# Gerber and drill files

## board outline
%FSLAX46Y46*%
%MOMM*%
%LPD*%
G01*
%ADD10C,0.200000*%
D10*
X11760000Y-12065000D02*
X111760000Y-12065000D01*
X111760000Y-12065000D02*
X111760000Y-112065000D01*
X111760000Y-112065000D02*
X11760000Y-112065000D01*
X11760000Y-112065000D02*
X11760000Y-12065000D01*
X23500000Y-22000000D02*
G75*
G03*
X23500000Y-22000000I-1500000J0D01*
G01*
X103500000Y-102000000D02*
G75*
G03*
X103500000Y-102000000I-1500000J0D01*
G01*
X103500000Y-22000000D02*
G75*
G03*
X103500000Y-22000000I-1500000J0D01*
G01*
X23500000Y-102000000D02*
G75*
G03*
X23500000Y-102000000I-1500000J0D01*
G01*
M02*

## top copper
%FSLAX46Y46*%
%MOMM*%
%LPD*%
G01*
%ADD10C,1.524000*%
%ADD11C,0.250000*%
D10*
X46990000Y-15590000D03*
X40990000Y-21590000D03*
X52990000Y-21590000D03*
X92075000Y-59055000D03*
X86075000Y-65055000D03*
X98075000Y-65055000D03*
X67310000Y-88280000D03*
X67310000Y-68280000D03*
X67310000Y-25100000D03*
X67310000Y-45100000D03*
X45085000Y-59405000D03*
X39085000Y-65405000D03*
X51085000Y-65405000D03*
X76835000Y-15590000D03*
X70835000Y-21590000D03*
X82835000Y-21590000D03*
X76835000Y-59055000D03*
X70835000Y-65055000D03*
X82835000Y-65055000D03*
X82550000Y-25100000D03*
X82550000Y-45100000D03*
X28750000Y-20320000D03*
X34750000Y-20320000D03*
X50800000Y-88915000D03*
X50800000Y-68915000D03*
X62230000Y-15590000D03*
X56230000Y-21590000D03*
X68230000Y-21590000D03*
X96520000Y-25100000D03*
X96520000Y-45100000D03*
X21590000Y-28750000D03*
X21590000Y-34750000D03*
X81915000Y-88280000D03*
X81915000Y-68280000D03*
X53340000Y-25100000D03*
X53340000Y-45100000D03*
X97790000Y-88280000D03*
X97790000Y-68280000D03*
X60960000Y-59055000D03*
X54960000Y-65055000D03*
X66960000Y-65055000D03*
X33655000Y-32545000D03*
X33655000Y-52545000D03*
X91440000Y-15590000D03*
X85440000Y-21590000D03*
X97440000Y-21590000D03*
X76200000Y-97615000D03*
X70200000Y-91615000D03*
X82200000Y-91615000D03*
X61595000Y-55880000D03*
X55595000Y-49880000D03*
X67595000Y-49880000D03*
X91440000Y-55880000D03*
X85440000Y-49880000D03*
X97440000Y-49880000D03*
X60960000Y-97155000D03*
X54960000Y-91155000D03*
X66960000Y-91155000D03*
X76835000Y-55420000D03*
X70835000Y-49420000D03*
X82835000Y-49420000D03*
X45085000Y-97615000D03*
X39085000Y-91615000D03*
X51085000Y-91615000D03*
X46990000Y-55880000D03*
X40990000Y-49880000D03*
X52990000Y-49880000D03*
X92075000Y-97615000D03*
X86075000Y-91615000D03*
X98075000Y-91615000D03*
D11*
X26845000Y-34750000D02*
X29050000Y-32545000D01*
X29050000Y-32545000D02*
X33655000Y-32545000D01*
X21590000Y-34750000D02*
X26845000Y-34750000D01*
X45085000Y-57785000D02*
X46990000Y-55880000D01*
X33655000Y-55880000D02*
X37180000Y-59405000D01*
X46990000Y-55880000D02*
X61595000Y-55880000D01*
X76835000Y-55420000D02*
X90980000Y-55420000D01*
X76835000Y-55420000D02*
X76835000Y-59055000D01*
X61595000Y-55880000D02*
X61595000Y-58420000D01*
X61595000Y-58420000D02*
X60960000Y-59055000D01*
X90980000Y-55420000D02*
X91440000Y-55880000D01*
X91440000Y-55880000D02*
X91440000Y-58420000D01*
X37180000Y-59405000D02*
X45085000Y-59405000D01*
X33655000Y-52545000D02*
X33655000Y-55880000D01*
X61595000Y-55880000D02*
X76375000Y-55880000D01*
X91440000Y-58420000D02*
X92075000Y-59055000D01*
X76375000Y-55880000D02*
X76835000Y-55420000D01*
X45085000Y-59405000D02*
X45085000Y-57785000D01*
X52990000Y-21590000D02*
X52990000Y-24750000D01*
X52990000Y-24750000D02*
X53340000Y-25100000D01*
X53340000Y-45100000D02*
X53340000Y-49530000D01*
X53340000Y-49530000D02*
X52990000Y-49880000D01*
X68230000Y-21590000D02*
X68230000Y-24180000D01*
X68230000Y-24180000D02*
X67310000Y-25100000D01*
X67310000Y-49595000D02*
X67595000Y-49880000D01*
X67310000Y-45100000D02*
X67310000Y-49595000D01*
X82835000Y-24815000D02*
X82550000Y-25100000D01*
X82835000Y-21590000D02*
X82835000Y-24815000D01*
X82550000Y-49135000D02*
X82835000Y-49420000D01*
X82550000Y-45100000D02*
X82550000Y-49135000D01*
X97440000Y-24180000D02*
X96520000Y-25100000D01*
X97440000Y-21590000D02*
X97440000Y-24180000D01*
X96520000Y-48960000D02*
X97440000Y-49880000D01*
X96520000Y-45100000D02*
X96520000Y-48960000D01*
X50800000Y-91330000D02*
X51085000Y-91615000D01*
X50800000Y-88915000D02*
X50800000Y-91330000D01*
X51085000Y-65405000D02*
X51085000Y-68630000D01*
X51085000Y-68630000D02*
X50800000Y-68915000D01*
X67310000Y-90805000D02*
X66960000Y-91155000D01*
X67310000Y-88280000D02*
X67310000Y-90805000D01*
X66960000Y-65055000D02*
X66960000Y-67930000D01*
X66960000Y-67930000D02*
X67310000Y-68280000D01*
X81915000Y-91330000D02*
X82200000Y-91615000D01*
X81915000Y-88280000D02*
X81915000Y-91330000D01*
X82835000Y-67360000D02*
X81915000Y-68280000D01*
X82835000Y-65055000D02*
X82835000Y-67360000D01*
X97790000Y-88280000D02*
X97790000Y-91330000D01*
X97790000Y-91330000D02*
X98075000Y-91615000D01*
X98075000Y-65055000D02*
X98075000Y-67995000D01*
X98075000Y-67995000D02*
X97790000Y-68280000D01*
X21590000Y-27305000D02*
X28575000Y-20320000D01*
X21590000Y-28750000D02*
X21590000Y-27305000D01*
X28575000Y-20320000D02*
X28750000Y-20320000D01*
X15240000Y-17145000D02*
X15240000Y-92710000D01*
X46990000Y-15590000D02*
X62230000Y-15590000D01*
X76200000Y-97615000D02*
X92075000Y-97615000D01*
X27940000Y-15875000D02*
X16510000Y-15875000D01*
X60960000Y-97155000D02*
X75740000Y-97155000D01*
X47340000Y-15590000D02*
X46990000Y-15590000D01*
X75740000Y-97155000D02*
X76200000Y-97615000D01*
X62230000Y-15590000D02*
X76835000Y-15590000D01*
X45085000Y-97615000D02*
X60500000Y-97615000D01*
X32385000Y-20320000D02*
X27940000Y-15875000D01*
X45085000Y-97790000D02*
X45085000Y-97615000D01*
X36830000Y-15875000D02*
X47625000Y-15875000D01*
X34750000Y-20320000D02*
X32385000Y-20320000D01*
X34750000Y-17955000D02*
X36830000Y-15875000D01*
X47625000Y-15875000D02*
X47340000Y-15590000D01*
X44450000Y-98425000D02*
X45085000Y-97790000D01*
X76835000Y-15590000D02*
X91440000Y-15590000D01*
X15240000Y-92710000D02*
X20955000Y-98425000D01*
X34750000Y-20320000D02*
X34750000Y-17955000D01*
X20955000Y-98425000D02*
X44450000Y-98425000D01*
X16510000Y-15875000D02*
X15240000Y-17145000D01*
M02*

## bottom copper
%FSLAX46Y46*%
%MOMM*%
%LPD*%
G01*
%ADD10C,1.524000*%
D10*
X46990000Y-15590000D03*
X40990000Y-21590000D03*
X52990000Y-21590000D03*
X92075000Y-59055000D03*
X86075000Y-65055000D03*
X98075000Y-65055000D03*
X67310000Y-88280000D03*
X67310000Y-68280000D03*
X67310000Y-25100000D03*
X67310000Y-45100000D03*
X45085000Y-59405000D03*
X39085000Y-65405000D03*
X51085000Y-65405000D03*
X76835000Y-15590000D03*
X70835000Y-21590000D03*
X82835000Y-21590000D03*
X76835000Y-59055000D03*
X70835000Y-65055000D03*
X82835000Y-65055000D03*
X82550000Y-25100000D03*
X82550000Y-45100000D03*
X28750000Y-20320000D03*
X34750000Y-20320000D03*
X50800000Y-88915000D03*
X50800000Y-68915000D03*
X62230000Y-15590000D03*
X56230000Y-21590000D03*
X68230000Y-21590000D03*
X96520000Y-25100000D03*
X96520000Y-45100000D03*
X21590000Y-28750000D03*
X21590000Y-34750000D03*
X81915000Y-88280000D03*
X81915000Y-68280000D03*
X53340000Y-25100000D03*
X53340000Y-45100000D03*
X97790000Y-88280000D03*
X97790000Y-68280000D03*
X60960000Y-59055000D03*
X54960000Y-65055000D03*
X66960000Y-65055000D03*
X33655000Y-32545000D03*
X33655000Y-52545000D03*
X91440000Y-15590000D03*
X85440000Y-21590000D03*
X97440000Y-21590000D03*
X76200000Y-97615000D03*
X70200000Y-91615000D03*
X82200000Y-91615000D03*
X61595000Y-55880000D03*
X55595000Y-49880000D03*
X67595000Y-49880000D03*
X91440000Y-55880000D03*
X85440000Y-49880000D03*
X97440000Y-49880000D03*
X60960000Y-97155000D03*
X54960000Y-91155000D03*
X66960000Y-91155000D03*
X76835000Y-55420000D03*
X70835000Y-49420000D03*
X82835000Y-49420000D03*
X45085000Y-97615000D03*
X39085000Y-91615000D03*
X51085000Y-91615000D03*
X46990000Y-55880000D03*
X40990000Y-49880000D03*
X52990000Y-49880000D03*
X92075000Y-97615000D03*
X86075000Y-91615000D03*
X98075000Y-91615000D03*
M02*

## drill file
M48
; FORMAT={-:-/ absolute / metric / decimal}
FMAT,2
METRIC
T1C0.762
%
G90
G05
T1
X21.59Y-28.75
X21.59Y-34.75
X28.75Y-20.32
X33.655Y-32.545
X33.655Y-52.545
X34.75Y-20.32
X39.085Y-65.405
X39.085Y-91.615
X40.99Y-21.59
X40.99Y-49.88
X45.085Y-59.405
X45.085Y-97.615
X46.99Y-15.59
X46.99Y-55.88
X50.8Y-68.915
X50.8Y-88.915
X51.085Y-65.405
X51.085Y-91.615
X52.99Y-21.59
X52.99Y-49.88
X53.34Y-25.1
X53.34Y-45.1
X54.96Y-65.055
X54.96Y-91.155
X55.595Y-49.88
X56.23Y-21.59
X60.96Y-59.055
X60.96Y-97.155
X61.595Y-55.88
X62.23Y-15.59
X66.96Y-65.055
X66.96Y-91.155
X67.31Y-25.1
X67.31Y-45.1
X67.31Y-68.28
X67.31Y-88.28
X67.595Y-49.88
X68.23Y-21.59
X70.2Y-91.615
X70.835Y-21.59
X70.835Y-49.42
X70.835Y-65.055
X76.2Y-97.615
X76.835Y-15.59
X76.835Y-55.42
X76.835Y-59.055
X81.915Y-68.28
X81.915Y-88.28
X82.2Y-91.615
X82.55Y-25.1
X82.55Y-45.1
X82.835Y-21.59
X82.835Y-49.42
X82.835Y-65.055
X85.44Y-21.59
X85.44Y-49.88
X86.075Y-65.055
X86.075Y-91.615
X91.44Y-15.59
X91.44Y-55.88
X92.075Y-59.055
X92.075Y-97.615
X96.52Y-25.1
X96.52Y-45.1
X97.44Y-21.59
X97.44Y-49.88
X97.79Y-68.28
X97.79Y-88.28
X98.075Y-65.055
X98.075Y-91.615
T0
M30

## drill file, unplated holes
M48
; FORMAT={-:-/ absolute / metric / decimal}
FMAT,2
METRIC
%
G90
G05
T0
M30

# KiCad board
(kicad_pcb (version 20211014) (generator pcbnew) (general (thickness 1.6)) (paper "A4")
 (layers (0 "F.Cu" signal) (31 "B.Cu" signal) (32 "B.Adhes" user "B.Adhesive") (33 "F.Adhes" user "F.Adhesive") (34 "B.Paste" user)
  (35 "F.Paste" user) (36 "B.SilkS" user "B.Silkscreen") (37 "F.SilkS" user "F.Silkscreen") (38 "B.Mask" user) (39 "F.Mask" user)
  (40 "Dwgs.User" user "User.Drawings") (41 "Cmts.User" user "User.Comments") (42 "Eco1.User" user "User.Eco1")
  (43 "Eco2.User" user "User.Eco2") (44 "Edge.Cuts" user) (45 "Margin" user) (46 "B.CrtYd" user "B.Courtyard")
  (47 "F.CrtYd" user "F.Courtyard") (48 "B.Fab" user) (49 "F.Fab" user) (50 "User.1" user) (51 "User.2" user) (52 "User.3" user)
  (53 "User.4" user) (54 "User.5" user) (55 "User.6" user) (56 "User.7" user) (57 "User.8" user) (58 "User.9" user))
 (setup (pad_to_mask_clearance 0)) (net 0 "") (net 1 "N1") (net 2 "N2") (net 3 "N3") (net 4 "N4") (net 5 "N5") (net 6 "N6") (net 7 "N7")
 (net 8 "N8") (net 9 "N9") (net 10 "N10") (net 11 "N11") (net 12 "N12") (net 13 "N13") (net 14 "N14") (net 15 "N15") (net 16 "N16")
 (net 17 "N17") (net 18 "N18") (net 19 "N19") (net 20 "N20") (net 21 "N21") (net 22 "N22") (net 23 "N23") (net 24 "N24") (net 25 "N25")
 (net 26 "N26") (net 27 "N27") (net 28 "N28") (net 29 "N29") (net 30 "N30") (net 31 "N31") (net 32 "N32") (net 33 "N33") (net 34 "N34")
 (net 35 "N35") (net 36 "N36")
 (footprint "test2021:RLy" (layer "F.Cu") (at 46.99 21.59)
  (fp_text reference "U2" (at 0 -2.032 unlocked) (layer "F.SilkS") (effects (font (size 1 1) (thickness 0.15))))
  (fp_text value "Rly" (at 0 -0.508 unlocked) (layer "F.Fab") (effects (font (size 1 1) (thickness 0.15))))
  (pad "1" thru_hole circle (at 0 -6) (size 1.524 1.524) (drill 0.762) (layers *.Cu *.Mask) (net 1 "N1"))
  (pad "2" thru_hole circle (at -6 0) (size 1.524 1.524) (drill 0.762) (layers *.Cu *.Mask) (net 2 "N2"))
  (pad "3" thru_hole circle (at 6 0) (size 1.524 1.524) (drill 0.762) (layers *.Cu *.Mask) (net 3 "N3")))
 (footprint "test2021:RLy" (layer "F.Cu") (at 92.075 65.055)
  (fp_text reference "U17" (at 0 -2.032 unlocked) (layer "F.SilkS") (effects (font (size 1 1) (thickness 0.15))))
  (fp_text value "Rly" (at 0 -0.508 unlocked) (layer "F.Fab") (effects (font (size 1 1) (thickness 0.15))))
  (pad "1" thru_hole circle (at 0 -6) (size 1.524 1.524) (drill 0.762) (layers *.Cu *.Mask) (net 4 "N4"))
  (pad "2" thru_hole circle (at -6 0) (size 1.524 1.524) (drill 0.762) (layers *.Cu *.Mask) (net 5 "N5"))
  (pad "3" thru_hole circle (at 6 0) (size 1.524 1.524) (drill 0.762) (layers *.Cu *.Mask) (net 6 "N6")))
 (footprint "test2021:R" (layer "F.Cu") (at 67.31 78.28 90)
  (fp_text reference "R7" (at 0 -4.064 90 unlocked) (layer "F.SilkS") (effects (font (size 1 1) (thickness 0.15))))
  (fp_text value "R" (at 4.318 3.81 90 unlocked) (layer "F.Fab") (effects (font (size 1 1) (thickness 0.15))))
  (pad "1" thru_hole circle (at -10 0 90) (size 1.524 1.524) (drill 0.762) (layers *.Cu *.Mask) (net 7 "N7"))
  (pad "2" thru_hole circle (at 10 0 90) (size 1.524 1.524) (drill 0.762) (layers *.Cu *.Mask) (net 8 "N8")))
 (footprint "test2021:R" (layer "F.Cu") (at 67.31 35.1 -90)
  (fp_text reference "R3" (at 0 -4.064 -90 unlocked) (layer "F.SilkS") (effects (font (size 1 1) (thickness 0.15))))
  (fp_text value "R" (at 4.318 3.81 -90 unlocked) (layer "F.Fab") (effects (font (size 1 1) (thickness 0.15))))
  (pad "1" thru_hole circle (at -10 0 270) (size 1.524 1.524) (drill 0.762) (layers *.Cu *.Mask) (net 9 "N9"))
  (pad "2" thru_hole circle (at 10 0 270) (size 1.524 1.524) (drill 0.762) (layers *.Cu *.Mask) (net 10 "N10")))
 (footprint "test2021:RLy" (layer "F.Cu") (at 45.085 65.405)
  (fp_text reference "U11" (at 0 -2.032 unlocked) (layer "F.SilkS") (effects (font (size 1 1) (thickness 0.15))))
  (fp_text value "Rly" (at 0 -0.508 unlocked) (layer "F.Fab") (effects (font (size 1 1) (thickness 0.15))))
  (pad "1" thru_hole circle (at 0 -6) (size 1.524 1.524) (drill 0.762) (layers *.Cu *.Mask) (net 4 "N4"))
  (pad "2" thru_hole circle (at -6 0) (size 1.524 1.524) (drill 0.762) (layers *.Cu *.Mask) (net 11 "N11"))
  (pad "3" thru_hole circle (at 6 0) (size 1.524 1.524) (drill 0.762) (layers *.Cu *.Mask) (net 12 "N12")))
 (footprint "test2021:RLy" (layer "F.Cu") (at 76.835 21.59)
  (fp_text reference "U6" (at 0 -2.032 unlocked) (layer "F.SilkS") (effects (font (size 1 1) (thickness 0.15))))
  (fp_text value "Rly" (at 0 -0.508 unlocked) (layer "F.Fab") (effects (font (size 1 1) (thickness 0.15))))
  (pad "1" thru_hole circle (at 0 -6) (size 1.524 1.524) (drill 0.762) (layers *.Cu *.Mask) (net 1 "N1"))
  (pad "2" thru_hole circle (at -6 0) (size 1.524 1.524) (drill 0.762) (layers *.Cu *.Mask) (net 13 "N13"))
  (pad "3" thru_hole circle (at 6 0) (size 1.524 1.524) (drill 0.762) (layers *.Cu *.Mask) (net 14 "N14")))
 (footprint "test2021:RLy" (layer "F.Cu") (at 76.835 65.055)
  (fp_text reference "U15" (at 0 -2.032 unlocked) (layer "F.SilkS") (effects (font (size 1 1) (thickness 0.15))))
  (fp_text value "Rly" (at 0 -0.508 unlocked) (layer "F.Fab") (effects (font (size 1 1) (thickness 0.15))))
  (pad "1" thru_hole circle (at 0 -6) (size 1.524 1.524) (drill 0.762) (layers *.Cu *.Mask) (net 4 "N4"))
  (pad "2" thru_hole circle (at -6 0) (size 1.524 1.524) (drill 0.762) (layers *.Cu *.Mask) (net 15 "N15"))
  (pad "3" thru_hole circle (at 6 0) (size 1.524 1.524) (drill 0.762) (layers *.Cu *.Mask) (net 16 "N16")))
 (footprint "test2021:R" (layer "F.Cu") (at 82.55 35.1 -90)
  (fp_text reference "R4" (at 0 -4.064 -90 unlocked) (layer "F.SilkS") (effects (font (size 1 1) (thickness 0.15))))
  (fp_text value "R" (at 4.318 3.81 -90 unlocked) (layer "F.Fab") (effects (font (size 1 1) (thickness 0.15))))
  (pad "1" thru_hole circle (at -10 0 270) (size 1.524 1.524) (drill 0.762) (layers *.Cu *.Mask) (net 14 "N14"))
  (pad "2" thru_hole circle (at 10 0 270) (size 1.524 1.524) (drill 0.762) (layers *.Cu *.Mask) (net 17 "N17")))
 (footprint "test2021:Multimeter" (layer "F.Cu") (at 31.75 20.32 90)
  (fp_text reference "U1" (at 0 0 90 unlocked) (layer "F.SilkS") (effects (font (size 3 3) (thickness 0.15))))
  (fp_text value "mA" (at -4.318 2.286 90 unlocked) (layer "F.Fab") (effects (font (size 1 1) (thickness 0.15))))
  (pad "1" thru_hole circle (at 0 -3 90) (size 1.524 1.524) (drill 0.762) (layers *.Cu *.Mask) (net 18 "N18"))
  (pad "2" thru_hole circle (at 0 3 90) (size 1.524 1.524) (drill 0.762) (layers *.Cu *.Mask) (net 1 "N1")))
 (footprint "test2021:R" (layer "F.Cu") (at 50.8 78.915 90)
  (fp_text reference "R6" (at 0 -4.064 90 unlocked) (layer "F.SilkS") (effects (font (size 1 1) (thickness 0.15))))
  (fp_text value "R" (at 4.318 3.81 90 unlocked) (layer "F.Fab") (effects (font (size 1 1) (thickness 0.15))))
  (pad "1" thru_hole circle (at -10 0 90) (size 1.524 1.524) (drill 0.762) (layers *.Cu *.Mask) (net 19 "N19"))
  (pad "2" thru_hole circle (at 10 0 90) (size 1.524 1.524) (drill 0.762) (layers *.Cu *.Mask) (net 12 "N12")))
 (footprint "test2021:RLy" (layer "F.Cu") (at 62.23 21.59)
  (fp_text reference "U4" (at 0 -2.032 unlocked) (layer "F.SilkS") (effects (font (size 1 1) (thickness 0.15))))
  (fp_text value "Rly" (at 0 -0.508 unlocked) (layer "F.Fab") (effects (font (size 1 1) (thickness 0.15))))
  (pad "1" thru_hole circle (at 0 -6) (size 1.524 1.524) (drill 0.762) (layers *.Cu *.Mask) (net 1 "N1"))
  (pad "2" thru_hole circle (at -6 0) (size 1.524 1.524) (drill 0.762) (layers *.Cu *.Mask) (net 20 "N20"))
  (pad "3" thru_hole circle (at 6 0) (size 1.524 1.524) (drill 0.762) (layers *.Cu *.Mask) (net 9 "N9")))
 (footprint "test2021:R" (layer "F.Cu") (at 96.52 35.1 -90)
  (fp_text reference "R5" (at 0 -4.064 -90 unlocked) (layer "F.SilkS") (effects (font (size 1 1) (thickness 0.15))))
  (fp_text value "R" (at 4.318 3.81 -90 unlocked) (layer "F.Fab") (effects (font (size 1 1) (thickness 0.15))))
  (pad "1" thru_hole circle (at -10 0 270) (size 1.524 1.524) (drill 0.762) (layers *.Cu *.Mask) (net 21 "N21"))
  (pad "2" thru_hole circle (at 10 0 270) (size 1.524 1.524) (drill 0.762) (layers *.Cu *.Mask) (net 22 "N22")))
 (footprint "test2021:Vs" (layer "F.Cu") (at 21.59 31.75)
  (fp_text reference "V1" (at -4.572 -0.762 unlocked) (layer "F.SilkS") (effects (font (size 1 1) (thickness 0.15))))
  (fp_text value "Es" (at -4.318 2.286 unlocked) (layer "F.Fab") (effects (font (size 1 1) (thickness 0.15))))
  (pad "1" thru_hole circle (at 0 -3) (size 1.524 1.524) (drill 0.762) (layers *.Cu *.Mask) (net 18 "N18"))
  (pad "2" thru_hole circle (at 0 3) (size 1.524 1.524) (drill 0.762) (layers *.Cu *.Mask) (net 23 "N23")))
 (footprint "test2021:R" (layer "F.Cu") (at 81.915 78.28 90)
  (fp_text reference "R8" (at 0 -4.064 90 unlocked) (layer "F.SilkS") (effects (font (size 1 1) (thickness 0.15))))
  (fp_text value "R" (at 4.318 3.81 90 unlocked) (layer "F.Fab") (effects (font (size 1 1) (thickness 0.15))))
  (pad "1" thru_hole circle (at -10 0 90) (size 1.524 1.524) (drill 0.762) (layers *.Cu *.Mask) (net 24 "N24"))
  (pad "2" thru_hole circle (at 10 0 90) (size 1.524 1.524) (drill 0.762) (layers *.Cu *.Mask) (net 16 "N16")))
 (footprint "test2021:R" (layer "F.Cu") (at 53.34 35.1 -90)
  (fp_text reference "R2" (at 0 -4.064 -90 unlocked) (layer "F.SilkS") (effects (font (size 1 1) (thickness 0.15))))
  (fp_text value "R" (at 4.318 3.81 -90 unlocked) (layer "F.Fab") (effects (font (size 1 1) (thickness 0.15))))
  (pad "1" thru_hole circle (at -10 0 270) (size 1.524 1.524) (drill 0.762) (layers *.Cu *.Mask) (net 3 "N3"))
  (pad "2" thru_hole circle (at 10 0 270) (size 1.524 1.524) (drill 0.762) (layers *.Cu *.Mask) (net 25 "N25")))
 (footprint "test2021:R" (layer "F.Cu") (at 97.79 78.28 90)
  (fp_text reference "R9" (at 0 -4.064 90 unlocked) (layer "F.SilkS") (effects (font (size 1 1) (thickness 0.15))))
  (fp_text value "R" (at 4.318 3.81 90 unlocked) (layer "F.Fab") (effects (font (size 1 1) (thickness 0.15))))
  (pad "1" thru_hole circle (at -10 0 90) (size 1.524 1.524) (drill 0.762) (layers *.Cu *.Mask) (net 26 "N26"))
  (pad "2" thru_hole circle (at 10 0 90) (size 1.524 1.524) (drill 0.762) (layers *.Cu *.Mask) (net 6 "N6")))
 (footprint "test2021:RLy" (layer "F.Cu") (at 60.96 65.055)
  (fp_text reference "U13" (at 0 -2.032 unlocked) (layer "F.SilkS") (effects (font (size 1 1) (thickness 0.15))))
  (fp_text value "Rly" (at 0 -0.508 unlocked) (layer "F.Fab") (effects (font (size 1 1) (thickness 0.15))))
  (pad "1" thru_hole circle (at 0 -6) (size 1.524 1.524) (drill 0.762) (layers *.Cu *.Mask) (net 4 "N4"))
  (pad "2" thru_hole circle (at -6 0) (size 1.524 1.524) (drill 0.762) (layers *.Cu *.Mask) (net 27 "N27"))
  (pad "3" thru_hole circle (at 6 0) (size 1.524 1.524) (drill 0.762) (layers *.Cu *.Mask) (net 8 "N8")))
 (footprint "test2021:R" (layer "F.Cu") (at 33.655 42.545 -90)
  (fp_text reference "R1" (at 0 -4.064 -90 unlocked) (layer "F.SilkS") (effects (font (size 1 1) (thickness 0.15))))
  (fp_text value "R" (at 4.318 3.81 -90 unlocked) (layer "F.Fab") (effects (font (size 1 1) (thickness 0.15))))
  (pad "1" thru_hole circle (at -10 0 270) (size 1.524 1.524) (drill 0.762) (layers *.Cu *.Mask) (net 23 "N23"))
  (pad "2" thru_hole circle (at 10 0 270) (size 1.524 1.524) (drill 0.762) (layers *.Cu *.Mask) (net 4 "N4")))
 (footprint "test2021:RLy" (layer "F.Cu") (at 91.44 21.59)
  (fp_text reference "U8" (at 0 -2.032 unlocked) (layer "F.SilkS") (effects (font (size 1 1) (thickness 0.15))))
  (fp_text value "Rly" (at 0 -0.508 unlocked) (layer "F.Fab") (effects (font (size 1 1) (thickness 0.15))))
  (pad "1" thru_hole circle (at 0 -6) (size 1.524 1.524) (drill 0.762) (layers *.Cu *.Mask) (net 1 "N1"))
  (pad "2" thru_hole circle (at -6 0) (size 1.524 1.524) (drill 0.762) (layers *.Cu *.Mask) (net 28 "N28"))
  (pad "3" thru_hole circle (at 6 0) (size 1.524 1.524) (drill 0.762) (layers *.Cu *.Mask) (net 21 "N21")))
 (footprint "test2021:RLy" (layer "B.Cu") (at 76.2 91.615)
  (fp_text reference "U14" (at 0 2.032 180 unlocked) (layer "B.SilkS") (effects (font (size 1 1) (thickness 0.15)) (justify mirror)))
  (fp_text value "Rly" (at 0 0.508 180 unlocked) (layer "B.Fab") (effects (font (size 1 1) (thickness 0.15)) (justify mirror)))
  (pad "1" thru_hole circle (at 0 6) (size 1.524 1.524) (drill 0.762) (layers *.Cu *.Mask) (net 1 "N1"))
  (pad "2" thru_hole circle (at -6 0) (size 1.524 1.524) (drill 0.762) (layers *.Cu *.Mask) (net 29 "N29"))
  (pad "3" thru_hole circle (at 6 0) (size 1.524 1.524) (drill 0.762) (layers *.Cu *.Mask) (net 24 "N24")))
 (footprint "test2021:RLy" (layer "B.Cu") (at 61.595 49.88)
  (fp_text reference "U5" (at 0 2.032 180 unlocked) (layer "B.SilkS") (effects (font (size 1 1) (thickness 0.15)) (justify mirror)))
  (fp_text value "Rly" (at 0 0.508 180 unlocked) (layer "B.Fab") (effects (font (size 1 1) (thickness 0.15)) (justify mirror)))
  (pad "1" thru_hole circle (at 0 6) (size 1.524 1.524) (drill 0.762) (layers *.Cu *.Mask) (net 4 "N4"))
  (pad "2" thru_hole circle (at -6 0) (size 1.524 1.524) (drill 0.762) (layers *.Cu *.Mask) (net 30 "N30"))
  (pad "3" thru_hole circle (at 6 0) (size 1.524 1.524) (drill 0.762) (layers *.Cu *.Mask) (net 10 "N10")))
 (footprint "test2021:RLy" (layer "B.Cu") (at 91.44 49.88)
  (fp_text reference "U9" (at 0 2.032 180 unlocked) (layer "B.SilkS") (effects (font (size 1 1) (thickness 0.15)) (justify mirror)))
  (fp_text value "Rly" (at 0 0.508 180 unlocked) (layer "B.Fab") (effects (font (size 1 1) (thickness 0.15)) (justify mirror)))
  (pad "1" thru_hole circle (at 0 6) (size 1.524 1.524) (drill 0.762) (layers *.Cu *.Mask) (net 4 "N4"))
  (pad "2" thru_hole circle (at -6 0) (size 1.524 1.524) (drill 0.762) (layers *.Cu *.Mask) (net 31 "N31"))
  (pad "3" thru_hole circle (at 6 0) (size 1.524 1.524) (drill 0.762) (layers *.Cu *.Mask) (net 22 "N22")))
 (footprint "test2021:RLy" (layer "B.Cu") (at 60.96 91.155)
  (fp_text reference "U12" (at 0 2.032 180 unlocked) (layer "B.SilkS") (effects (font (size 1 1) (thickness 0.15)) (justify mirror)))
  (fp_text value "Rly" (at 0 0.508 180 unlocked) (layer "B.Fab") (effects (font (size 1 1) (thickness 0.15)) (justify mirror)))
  (pad "1" thru_hole circle (at 0 6) (size 1.524 1.524) (drill 0.762) (layers *.Cu *.Mask) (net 1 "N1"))
  (pad "2" thru_hole circle (at -6 0) (size 1.524 1.524) (drill 0.762) (layers *.Cu *.Mask) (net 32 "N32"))
  (pad "3" thru_hole circle (at 6 0) (size 1.524 1.524) (drill 0.762) (layers *.Cu *.Mask) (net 7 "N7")))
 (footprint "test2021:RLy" (layer "B.Cu") (at 76.835 49.42)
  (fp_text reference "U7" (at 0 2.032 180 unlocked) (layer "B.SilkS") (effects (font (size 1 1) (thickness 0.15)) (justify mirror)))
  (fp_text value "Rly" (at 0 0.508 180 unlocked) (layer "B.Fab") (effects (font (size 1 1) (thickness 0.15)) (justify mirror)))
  (pad "1" thru_hole circle (at 0 6) (size 1.524 1.524) (drill 0.762) (layers *.Cu *.Mask) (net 4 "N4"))
  (pad "2" thru_hole circle (at -6 0) (size 1.524 1.524) (drill 0.762) (layers *.Cu *.Mask) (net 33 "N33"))
  (pad "3" thru_hole circle (at 6 0) (size 1.524 1.524) (drill 0.762) (layers *.Cu *.Mask) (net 17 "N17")))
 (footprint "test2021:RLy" (layer "B.Cu") (at 45.085 91.615)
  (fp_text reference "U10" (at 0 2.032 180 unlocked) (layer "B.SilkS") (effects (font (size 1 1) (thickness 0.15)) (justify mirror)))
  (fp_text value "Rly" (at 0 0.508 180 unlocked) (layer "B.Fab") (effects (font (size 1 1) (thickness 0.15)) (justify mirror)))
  (pad "1" thru_hole circle (at 0 6) (size 1.524 1.524) (drill 0.762) (layers *.Cu *.Mask) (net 1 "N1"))
  (pad "2" thru_hole circle (at -6 0) (size 1.524 1.524) (drill 0.762) (layers *.Cu *.Mask) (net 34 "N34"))
  (pad "3" thru_hole circle (at 6 0) (size 1.524 1.524) (drill 0.762) (layers *.Cu *.Mask) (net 19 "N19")))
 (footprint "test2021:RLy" (layer "B.Cu") (at 46.99 49.88)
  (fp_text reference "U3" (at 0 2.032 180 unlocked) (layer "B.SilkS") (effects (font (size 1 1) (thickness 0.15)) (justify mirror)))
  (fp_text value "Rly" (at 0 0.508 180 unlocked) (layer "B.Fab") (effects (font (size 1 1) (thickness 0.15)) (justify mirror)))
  (pad "1" thru_hole circle (at 0 6) (size 1.524 1.524) (drill 0.762) (layers *.Cu *.Mask) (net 4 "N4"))
  (pad "2" thru_hole circle (at -6 0) (size 1.524 1.524) (drill 0.762) (layers *.Cu *.Mask) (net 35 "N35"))
  (pad "3" thru_hole circle (at 6 0) (size 1.524 1.524) (drill 0.762) (layers *.Cu *.Mask) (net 25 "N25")))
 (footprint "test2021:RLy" (layer "B.Cu") (at 92.075 91.615)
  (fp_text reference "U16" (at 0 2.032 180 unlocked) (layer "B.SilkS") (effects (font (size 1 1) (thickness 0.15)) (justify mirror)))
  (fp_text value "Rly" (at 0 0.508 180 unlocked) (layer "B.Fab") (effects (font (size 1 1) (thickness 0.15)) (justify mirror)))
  (pad "1" thru_hole circle (at 0 6) (size 1.524 1.524) (drill 0.762) (layers *.Cu *.Mask) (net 1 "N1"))
  (pad "2" thru_hole circle (at -6 0) (size 1.524 1.524) (drill 0.762) (layers *.Cu *.Mask) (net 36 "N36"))
  (pad "3" thru_hole circle (at 6 0) (size 1.524 1.524) (drill 0.762) (layers *.Cu *.Mask) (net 26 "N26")))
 (gr_rect (start 11.76 12.065) (end 111.76 112.065) (layer "Edge.Cuts") (width 0.2) (fill none))
 (gr_circle (center 22 22) (end 23.5 22) (layer "Edge.Cuts") (width 0.2) (fill none))
 (gr_circle (center 102 102) (end 103.5 102) (layer "Edge.Cuts") (width 0.2) (fill none))
 (gr_circle (center 102 22) (end 103.5 22) (layer "Edge.Cuts") (width 0.2) (fill none))
 (gr_circle (center 22 102) (end 23.5 102) (layer "Edge.Cuts") (width 0.2) (fill none))
 (segment (start 26.845 34.75) (end 29.05 32.545) (width 0.25) (layer "F.Cu") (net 23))
 (segment (start 29.05 32.545) (end 33.655 32.545) (width 0.25) (layer "F.Cu") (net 23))
 (segment (start 21.59 34.75) (end 26.845 34.75) (width 0.25) (layer "F.Cu") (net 23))
 (segment (start 45.085 57.785) (end 46.99 55.88) (width 0.25) (layer "F.Cu") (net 4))
 (segment (start 33.655 55.88) (end 37.18 59.405) (width 0.25) (layer "F.Cu") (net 4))
 (segment (start 46.99 55.88) (end 61.595 55.88) (width 0.25) (layer "F.Cu") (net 4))
 (segment (start 76.835 55.42) (end 90.98 55.42) (width 0.25) (layer "F.Cu") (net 4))
 (segment (start 76.835 55.42) (end 76.835 59.055) (width 0.25) (layer "F.Cu") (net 4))
 (segment (start 61.595 55.88) (end 61.595 58.42) (width 0.25) (layer "F.Cu") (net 4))
 (segment (start 61.595 58.42) (end 60.96 59.055) (width 0.25) (layer "F.Cu") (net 4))
 (segment (start 90.98 55.42) (end 91.44 55.88) (width 0.25) (layer "F.Cu") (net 4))
 (segment (start 91.44 55.88) (end 91.44 58.42) (width 0.25) (layer "F.Cu") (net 4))
 (segment (start 37.18 59.405) (end 45.085 59.405) (width 0.25) (layer "F.Cu") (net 4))
 (segment (start 33.655 52.545) (end 33.655 55.88) (width 0.25) (layer "F.Cu") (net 4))
 (segment (start 61.595 55.88) (end 76.375 55.88) (width 0.25) (layer "F.Cu") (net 4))
 (segment (start 91.44 58.42) (end 92.075 59.055) (width 0.25) (layer "F.Cu") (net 4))
 (segment (start 76.375 55.88) (end 76.835 55.42) (width 0.25) (layer "F.Cu") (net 4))
 (segment (start 45.085 59.405) (end 45.085 57.785) (width 0.25) (layer "F.Cu") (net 4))
 (segment (start 52.99 21.59) (end 52.99 24.75) (width 0.25) (layer "F.Cu") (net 3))
 (segment (start 52.99 24.75) (end 53.34 25.1) (width 0.25) (layer "F.Cu") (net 3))
 (segment (start 53.34 45.1) (end 53.34 49.53) (width 0.25) (layer "F.Cu") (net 25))
 (segment (start 53.34 49.53) (end 52.99 49.88) (width 0.25) (layer "F.Cu") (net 25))
 (segment (start 68.23 21.59) (end 68.23 24.18) (width 0.25) (layer "F.Cu") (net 9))
 (segment (start 68.23 24.18) (end 67.31 25.1) (width 0.25) (layer "F.Cu") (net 9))
 (segment (start 67.31 49.595) (end 67.595 49.88) (width 0.25) (layer "F.Cu") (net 10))
 (segment (start 67.31 45.1) (end 67.31 49.595) (width 0.25) (layer "F.Cu") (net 10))
 (segment (start 82.835 24.815) (end 82.55 25.1) (width 0.25) (layer "F.Cu") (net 14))
 (segment (start 82.835 21.59) (end 82.835 24.815) (width 0.25) (layer "F.Cu") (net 14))
 (segment (start 82.55 49.135) (end 82.835 49.42) (width 0.25) (layer "F.Cu") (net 17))
 (segment (start 82.55 45.1) (end 82.55 49.135) (width 0.25) (layer "F.Cu") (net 17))
 (segment (start 97.44 24.18) (end 96.52 25.1) (width 0.25) (layer "F.Cu") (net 21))
 (segment (start 97.44 21.59) (end 97.44 24.18) (width 0.25) (layer "F.Cu") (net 21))
 (segment (start 96.52 48.96) (end 97.44 49.88) (width 0.25) (layer "F.Cu") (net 22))
 (segment (start 96.52 45.1) (end 96.52 48.96) (width 0.25) (layer "F.Cu") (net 22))
 (segment (start 50.8 91.33) (end 51.085 91.615) (width 0.25) (layer "F.Cu") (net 19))
 (segment (start 50.8 88.915) (end 50.8 91.33) (width 0.25) (layer "F.Cu") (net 19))
 (segment (start 51.085 65.405) (end 51.085 68.63) (width 0.25) (layer "F.Cu") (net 12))
 (segment (start 51.085 68.63) (end 50.8 68.915) (width 0.25) (layer "F.Cu") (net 12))
 (segment (start 67.31 90.805) (end 66.96 91.155) (width 0.25) (layer "F.Cu") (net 7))
 (segment (start 67.31 88.28) (end 67.31 90.805) (width 0.25) (layer "F.Cu") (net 7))
 (segment (start 66.96 65.055) (end 66.96 67.93) (width 0.25) (layer "F.Cu") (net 8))
 (segment (start 66.96 67.93) (end 67.31 68.28) (width 0.25) (layer "F.Cu") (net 8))
 (segment (start 81.915 91.33) (end 82.2 91.615) (width 0.25) (layer "F.Cu") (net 24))
 (segment (start 81.915 88.28) (end 81.915 91.33) (width 0.25) (layer "F.Cu") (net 24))
 (segment (start 82.835 67.36) (end 81.915 68.28) (width 0.25) (layer "F.Cu") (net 16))
 (segment (start 82.835 65.055) (end 82.835 67.36) (width 0.25) (layer "F.Cu") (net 16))
 (segment (start 97.79 88.28) (end 97.79 91.33) (width 0.25) (layer "F.Cu") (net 26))
 (segment (start 97.79 91.33) (end 98.075 91.615) (width 0.25) (layer "F.Cu") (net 26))
 (segment (start 98.075 65.055) (end 98.075 67.995) (width 0.25) (layer "F.Cu") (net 6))
 (segment (start 98.075 67.995) (end 97.79 68.28) (width 0.25) (layer "F.Cu") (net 6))
 (segment (start 21.59 27.305) (end 28.575 20.32) (width 0.25) (layer "F.Cu") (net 18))
 (segment (start 21.59 28.75) (end 21.59 27.305) (width 0.25) (layer "F.Cu") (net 18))
 (segment (start 28.575 20.32) (end 28.75 20.32) (width 0.25) (layer "F.Cu") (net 18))
 (segment (start 15.24 17.145) (end 15.24 92.71) (width 0.25) (layer "F.Cu") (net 1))
 (segment (start 46.99 15.59) (end 62.23 15.59) (width 0.25) (layer "F.Cu") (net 1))
 (segment (start 76.2 97.615) (end 92.075 97.615) (width 0.25) (layer "F.Cu") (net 1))
 (segment (start 27.94 15.875) (end 16.51 15.875) (width 0.25) (layer "F.Cu") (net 1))
 (segment (start 60.96 97.155) (end 75.74 97.155) (width 0.25) (layer "F.Cu") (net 1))
 (segment (start 47.34 15.59) (end 46.99 15.59) (width 0.25) (layer "F.Cu") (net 1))
 (segment (start 75.74 97.155) (end 76.2 97.615) (width 0.25) (layer "F.Cu") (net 1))
 (segment (start 62.23 15.59) (end 76.835 15.59) (width 0.25) (layer "F.Cu") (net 1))
 (segment (start 45.085 97.615) (end 60.5 97.615) (width 0.25) (layer "F.Cu") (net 1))
 (segment (start 32.385 20.32) (end 27.94 15.875) (width 0.25) (layer "F.Cu") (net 1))
 (segment (start 45.085 97.79) (end 45.085 97.615) (width 0.25) (layer "F.Cu") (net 1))
 (segment (start 36.83 15.875) (end 47.625 15.875) (width 0.25) (layer "F.Cu") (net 1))
 (segment (start 34.75 20.32) (end 32.385 20.32) (width 0.25) (layer "F.Cu") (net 1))
 (segment (start 34.75 17.955) (end 36.83 15.875) (width 0.25) (layer "F.Cu") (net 1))
 (segment (start 47.625 15.875) (end 47.34 15.59) (width 0.25) (layer "F.Cu") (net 1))
 (segment (start 44.45 98.425) (end 45.085 97.79) (width 0.25) (layer "F.Cu") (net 1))
 (segment (start 76.835 15.59) (end 91.44 15.59) (width 0.25) (layer "F.Cu") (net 1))
 (segment (start 15.24 92.71) (end 20.955 98.425) (width 0.25) (layer "F.Cu") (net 1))
 (segment (start 34.75 20.32) (end 34.75 17.955) (width 0.25) (layer "F.Cu") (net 1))
 (segment (start 20.955 98.425) (end 44.45 98.425) (width 0.25) (layer "F.Cu") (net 1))
 (segment (start 16.51 15.875) (end 15.24 17.145) (width 0.25) (layer "F.Cu") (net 1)))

